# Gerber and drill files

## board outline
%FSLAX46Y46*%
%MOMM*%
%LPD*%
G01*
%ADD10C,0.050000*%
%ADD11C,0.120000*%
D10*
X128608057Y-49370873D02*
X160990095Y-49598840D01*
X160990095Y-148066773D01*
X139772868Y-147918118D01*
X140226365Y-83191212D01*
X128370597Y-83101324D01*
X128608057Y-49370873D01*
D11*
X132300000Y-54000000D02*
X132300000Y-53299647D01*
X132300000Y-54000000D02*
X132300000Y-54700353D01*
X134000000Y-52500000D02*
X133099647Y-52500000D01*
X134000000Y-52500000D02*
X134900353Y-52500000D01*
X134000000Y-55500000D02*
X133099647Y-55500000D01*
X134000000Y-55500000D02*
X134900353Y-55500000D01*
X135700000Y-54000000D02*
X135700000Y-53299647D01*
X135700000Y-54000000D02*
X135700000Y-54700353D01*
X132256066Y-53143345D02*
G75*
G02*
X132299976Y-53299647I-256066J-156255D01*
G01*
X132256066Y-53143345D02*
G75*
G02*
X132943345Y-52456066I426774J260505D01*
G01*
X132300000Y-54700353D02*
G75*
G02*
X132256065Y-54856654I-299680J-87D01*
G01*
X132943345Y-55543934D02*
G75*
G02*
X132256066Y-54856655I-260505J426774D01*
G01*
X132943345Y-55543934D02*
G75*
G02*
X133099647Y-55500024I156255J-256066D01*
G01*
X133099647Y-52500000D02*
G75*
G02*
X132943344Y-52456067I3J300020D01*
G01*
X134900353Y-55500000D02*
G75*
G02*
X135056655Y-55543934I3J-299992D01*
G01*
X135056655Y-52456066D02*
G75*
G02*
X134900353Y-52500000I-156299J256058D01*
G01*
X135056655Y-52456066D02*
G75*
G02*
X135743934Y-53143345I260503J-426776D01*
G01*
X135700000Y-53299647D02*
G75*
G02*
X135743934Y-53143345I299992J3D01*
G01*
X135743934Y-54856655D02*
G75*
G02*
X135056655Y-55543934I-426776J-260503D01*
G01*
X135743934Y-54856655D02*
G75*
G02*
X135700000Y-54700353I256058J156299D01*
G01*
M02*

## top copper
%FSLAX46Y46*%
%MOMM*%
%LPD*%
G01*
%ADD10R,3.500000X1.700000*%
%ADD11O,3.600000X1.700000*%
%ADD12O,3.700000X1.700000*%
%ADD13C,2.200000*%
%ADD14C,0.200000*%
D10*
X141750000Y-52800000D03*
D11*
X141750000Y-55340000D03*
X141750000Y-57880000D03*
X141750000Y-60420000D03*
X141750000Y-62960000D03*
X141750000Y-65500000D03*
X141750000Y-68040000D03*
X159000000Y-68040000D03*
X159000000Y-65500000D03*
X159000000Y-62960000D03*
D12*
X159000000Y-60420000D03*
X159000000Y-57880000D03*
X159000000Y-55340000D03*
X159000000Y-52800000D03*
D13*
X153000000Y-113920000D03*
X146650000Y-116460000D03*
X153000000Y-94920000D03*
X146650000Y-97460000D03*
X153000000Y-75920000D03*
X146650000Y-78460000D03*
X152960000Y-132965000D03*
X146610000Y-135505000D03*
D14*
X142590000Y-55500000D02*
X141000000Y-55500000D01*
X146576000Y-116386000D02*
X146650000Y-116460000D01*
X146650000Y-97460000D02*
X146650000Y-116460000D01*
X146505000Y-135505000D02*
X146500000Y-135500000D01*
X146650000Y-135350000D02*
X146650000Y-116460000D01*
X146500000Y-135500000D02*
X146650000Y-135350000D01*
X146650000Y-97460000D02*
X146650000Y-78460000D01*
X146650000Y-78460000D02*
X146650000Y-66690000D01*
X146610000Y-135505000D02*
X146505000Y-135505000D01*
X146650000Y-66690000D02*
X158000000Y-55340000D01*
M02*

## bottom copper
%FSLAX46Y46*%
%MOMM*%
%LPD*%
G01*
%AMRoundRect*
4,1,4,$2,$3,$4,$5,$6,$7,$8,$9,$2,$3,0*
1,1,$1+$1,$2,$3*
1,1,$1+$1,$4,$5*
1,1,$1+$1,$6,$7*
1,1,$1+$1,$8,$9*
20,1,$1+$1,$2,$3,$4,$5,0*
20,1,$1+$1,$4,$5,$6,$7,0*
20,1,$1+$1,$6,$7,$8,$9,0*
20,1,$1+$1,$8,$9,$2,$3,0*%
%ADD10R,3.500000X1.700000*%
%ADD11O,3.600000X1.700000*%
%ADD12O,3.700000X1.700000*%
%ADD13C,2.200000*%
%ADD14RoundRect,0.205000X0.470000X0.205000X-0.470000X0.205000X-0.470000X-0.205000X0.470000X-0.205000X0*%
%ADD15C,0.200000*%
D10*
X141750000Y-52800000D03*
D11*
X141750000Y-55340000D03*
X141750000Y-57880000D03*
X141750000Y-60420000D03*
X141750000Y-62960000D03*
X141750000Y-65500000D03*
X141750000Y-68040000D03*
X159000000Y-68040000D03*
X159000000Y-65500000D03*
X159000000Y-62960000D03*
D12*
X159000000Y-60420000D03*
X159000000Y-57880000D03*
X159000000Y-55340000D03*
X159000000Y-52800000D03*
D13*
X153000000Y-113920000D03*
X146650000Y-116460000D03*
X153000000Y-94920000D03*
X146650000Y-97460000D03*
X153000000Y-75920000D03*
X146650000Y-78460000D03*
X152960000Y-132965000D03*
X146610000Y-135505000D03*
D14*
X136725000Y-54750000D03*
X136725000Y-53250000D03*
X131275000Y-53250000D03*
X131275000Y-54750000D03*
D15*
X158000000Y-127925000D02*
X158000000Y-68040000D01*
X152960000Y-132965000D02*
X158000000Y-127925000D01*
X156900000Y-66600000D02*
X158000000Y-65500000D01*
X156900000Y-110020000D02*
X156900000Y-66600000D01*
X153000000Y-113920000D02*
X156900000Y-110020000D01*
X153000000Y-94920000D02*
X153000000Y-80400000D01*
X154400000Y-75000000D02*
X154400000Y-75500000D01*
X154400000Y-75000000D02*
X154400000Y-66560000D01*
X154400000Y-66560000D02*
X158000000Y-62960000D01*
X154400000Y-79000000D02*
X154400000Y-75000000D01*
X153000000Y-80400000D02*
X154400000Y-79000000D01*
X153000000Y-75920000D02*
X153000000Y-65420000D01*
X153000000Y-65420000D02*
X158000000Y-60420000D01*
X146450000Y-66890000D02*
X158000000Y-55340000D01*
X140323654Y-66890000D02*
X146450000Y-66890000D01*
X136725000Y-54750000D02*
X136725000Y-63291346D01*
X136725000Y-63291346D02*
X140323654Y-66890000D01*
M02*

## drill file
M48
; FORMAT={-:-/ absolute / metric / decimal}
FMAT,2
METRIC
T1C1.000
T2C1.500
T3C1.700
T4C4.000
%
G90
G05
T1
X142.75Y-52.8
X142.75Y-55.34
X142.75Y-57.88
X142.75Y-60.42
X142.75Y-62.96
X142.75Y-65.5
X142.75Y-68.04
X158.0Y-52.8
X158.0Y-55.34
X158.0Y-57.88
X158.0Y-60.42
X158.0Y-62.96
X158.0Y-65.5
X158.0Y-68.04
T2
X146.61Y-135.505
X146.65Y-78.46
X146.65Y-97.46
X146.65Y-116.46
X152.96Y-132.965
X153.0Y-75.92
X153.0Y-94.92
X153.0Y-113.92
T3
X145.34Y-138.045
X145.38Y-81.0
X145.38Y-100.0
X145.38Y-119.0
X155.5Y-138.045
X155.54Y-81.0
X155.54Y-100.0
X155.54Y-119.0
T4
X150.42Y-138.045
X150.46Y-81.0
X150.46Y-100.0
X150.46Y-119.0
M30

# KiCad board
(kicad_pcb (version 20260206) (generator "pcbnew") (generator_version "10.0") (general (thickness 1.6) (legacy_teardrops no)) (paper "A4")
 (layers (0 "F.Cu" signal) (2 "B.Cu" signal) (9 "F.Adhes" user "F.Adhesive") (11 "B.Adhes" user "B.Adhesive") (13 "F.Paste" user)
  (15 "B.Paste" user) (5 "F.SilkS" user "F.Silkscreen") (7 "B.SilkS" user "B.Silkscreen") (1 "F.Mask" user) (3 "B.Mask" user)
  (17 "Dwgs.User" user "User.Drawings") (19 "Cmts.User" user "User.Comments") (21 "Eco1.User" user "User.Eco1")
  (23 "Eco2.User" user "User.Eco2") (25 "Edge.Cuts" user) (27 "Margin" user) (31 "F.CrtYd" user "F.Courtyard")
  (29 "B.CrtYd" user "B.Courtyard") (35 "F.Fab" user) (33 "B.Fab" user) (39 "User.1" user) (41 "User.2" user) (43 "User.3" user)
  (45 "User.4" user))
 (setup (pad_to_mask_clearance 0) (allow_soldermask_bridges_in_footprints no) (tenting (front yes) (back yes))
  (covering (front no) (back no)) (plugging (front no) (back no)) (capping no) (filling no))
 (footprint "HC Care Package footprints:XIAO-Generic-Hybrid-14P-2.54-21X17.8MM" (layer "F.Cu") (at 150.375 60.42)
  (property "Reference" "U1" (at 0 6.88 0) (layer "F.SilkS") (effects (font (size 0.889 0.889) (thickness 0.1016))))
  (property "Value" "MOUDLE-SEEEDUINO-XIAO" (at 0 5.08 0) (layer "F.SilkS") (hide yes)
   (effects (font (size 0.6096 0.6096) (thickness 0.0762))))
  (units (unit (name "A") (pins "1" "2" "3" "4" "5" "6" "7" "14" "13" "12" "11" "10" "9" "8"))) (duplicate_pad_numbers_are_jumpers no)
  (pad "1" thru_hole rect (at -7.625 -7.62) (size 3.5 1.7) (drill 1 (offset -1 0)) (layers "*.Cu" "*.Mask") (remove_unused_layers no)
   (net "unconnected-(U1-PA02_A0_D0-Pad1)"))
  (pad "2" thru_hole oval (at -7.625 -5.08) (size 3.6 1.7) (drill 1 (offset -1 0)) (layers "*.Cu" "*.Mask") (remove_unused_layers no)
   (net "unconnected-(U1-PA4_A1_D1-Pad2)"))
  (pad "3" thru_hole oval (at -7.625 -2.54) (size 3.6 1.7) (drill 1 (offset -1 0)) (layers "*.Cu" "*.Mask") (remove_unused_layers no)
   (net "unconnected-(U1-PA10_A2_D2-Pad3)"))
  (pad "4" thru_hole oval (at -7.625 0) (size 3.6 1.7) (drill 1 (offset -1 0)) (layers "*.Cu" "*.Mask") (remove_unused_layers no)
   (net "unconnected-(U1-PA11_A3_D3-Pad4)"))
  (pad "5" thru_hole oval (at -7.625 2.54) (size 3.6 1.7) (drill 1 (offset -1 0)) (layers "*.Cu" "*.Mask") (remove_unused_layers no)
   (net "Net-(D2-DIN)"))
  (pad "6" thru_hole oval (at -7.625 5.08 180) (size 3.6 1.7) (drill 1 (offset 1 0)) (layers "*.Cu" "*.Mask") (remove_unused_layers no)
   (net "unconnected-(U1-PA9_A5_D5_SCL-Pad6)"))
  (pad "7" thru_hole oval (at -7.625 7.62) (size 3.6 1.7) (drill 1 (offset -1 0)) (layers "*.Cu" "*.Mask") (remove_unused_layers no)
   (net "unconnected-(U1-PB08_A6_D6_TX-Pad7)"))
  (pad "8" thru_hole oval (at 7.625 7.62) (size 3.6 1.7) (drill 1 (offset 1 0)) (layers "*.Cu" "*.Mask") (remove_unused_layers no)
   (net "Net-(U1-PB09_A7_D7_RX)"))
  (pad "9" thru_hole oval (at 7.625 5.08) (size 3.6 1.7) (drill 1 (offset 1 0)) (layers "*.Cu" "*.Mask") (remove_unused_layers no)
   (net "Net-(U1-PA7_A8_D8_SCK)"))
  (pad "10" thru_hole oval (at 7.625 2.54) (size 3.6 1.7) (drill 1 (offset 1 0)) (layers "*.Cu" "*.Mask") (remove_unused_layers no)
   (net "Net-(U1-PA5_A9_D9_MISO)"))
  (pad "11" thru_hole oval (at 7.625 0) (size 3.7 1.7) (drill 1 (offset 1 0)) (layers "*.Cu" "*.Mask") (remove_unused_layers no)
   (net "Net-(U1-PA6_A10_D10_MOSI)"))
  (pad "12" thru_hole oval (at 7.625 -2.54) (size 3.7 1.7) (drill 1 (offset 1 0)) (layers "*.Cu" "*.Mask") (remove_unused_layers no)
   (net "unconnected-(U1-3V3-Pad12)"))
  (pad "13" thru_hole oval (at 7.625 -5.08) (size 3.7 1.7) (drill 1 (offset 1 0)) (layers "*.Cu" "*.Mask") (remove_unused_layers no)
   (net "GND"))
  (pad "14" thru_hole oval (at 7.625 -7.62) (size 3.7 1.7) (drill 1 (offset 1 0)) (layers "*.Cu" "*.Mask") (remove_unused_layers no)
   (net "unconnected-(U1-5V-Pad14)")))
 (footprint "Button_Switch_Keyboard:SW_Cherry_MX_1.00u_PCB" (layer "F.Cu") (at 153 113.92)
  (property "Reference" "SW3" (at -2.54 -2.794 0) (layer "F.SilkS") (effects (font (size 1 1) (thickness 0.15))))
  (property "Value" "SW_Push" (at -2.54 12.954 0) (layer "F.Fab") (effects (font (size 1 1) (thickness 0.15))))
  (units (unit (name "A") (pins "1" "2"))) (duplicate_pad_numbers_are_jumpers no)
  (pad "" np_thru_hole circle (at -7.62 5.08) (size 1.7 1.7) (drill 1.7) (layers "*.Cu" "*.Mask"))
  (pad "" np_thru_hole circle (at -2.54 5.08) (size 4 4) (drill 4) (layers "*.Cu" "*.Mask"))
  (pad "" np_thru_hole circle (at 2.54 5.08) (size 1.7 1.7) (drill 1.7) (layers "*.Cu" "*.Mask"))
  (pad "1" thru_hole circle (at 0 0) (size 2.2 2.2) (drill 1.5) (layers "*.Cu" "*.Mask") (remove_unused_layers no)
   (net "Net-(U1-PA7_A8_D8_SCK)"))
  (pad "2" thru_hole circle (at -6.35 2.54) (size 2.2 2.2) (drill 1.5) (layers "*.Cu" "*.Mask") (remove_unused_layers no) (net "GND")))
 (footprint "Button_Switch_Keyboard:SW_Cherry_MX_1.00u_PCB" (layer "F.Cu") (at 153 94.92)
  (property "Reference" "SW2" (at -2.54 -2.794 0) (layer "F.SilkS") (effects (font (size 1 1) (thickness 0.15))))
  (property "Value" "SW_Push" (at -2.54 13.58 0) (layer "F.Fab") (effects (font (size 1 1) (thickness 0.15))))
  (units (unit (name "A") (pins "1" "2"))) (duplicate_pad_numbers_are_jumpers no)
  (pad "" np_thru_hole circle (at -7.62 5.08) (size 1.7 1.7) (drill 1.7) (layers "*.Cu" "*.Mask"))
  (pad "" np_thru_hole circle (at -2.54 5.08) (size 4 4) (drill 4) (layers "*.Cu" "*.Mask"))
  (pad "" np_thru_hole circle (at 2.54 5.08) (size 1.7 1.7) (drill 1.7) (layers "*.Cu" "*.Mask"))
  (pad "1" thru_hole circle (at 0 0) (size 2.2 2.2) (drill 1.5) (layers "*.Cu" "*.Mask") (remove_unused_layers no)
   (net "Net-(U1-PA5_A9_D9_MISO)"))
  (pad "2" thru_hole circle (at -6.35 2.54) (size 2.2 2.2) (drill 1.5) (layers "*.Cu" "*.Mask") (remove_unused_layers no) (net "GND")))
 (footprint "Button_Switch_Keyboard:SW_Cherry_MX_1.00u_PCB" (layer "F.Cu") (at 153 75.92)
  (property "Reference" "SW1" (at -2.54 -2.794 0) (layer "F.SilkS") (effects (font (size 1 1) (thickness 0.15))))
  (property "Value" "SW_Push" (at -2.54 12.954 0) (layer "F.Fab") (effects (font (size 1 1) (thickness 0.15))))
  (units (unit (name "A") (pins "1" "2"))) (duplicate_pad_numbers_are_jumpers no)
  (pad "" np_thru_hole circle (at -7.62 5.08) (size 1.7 1.7) (drill 1.7) (layers "*.Cu" "*.Mask"))
  (pad "" np_thru_hole circle (at -2.54 5.08) (size 4 4) (drill 4) (layers "*.Cu" "*.Mask"))
  (pad "" np_thru_hole circle (at 2.54 5.08) (size 1.7 1.7) (drill 1.7) (layers "*.Cu" "*.Mask"))
  (pad "1" thru_hole circle (at 0 0) (size 2.2 2.2) (drill 1.5) (layers "*.Cu" "*.Mask") (remove_unused_layers no)
   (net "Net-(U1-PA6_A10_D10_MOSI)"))
  (pad "2" thru_hole circle (at -6.35 2.54) (size 2.2 2.2) (drill 1.5) (layers "*.Cu" "*.Mask") (remove_unused_layers no) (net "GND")))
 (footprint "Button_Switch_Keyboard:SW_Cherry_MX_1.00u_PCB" (layer "F.Cu") (at 152.96 132.965)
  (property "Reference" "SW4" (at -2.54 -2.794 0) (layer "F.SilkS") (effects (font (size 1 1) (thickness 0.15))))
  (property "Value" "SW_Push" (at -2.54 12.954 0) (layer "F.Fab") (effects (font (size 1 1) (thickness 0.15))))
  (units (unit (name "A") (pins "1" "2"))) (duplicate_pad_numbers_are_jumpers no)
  (pad "" np_thru_hole circle (at -7.62 5.08) (size 1.7 1.7) (drill 1.7) (layers "*.Cu" "*.Mask"))
  (pad "" np_thru_hole circle (at -2.54 5.08) (size 4 4) (drill 4) (layers "*.Cu" "*.Mask"))
  (pad "" np_thru_hole circle (at 2.54 5.08) (size 1.7 1.7) (drill 1.7) (layers "*.Cu" "*.Mask"))
  (pad "1" thru_hole circle (at 0 0) (size 2.2 2.2) (drill 1.5) (layers "*.Cu" "*.Mask") (remove_unused_layers no)
   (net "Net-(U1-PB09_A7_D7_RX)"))
  (pad "2" thru_hole circle (at -6.35 2.54) (size 2.2 2.2) (drill 1.5) (layers "*.Cu" "*.Mask") (remove_unused_layers no) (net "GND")))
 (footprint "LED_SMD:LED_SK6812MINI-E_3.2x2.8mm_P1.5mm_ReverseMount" (layer "B.Cu") (at 134 54 180)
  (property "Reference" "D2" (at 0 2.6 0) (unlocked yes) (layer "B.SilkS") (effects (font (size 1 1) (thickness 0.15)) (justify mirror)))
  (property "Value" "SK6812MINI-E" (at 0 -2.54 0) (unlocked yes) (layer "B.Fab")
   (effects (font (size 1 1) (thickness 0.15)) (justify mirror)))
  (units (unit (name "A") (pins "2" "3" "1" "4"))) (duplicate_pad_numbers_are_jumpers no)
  (fp_line (start 1.7 0) (end 1.7 0.700353) (stroke (width 0.12) (type solid)) (layer "Edge.Cuts"))
  (fp_line (start 1.7 0) (end 1.7 -0.700353) (stroke (width 0.12) (type solid)) (layer "Edge.Cuts"))
  (fp_line (start 0 1.5) (end 0.900353 1.5) (stroke (width 0.12) (type solid)) (layer "Edge.Cuts"))
  (fp_line (start 0 1.5) (end -0.900353 1.5) (stroke (width 0.12) (type solid)) (layer "Edge.Cuts"))
  (fp_line (start 0 -1.5) (end 0.900353 -1.5) (stroke (width 0.12) (type solid)) (layer "Edge.Cuts"))
  (fp_line (start 0 -1.5) (end -0.900353 -1.5) (stroke (width 0.12) (type solid)) (layer "Edge.Cuts"))
  (fp_line (start -1.7 0) (end -1.7 0.700353) (stroke (width 0.12) (type solid)) (layer "Edge.Cuts"))
  (fp_line (start -1.7 0) (end -1.7 -0.700353) (stroke (width 0.12) (type solid)) (layer "Edge.Cuts"))
  (fp_arc (start 1.743934 0.856655) (mid 1.711191 0.781533) (end 1.7 0.700353) (stroke (width 0.12) (type solid)) (layer "Edge.Cuts"))
  (fp_arc (start 1.743934 0.856655) (mid 1.670713 1.470713) (end 1.056655 1.543934) (stroke (width 0.12) (type solid)) (layer "Edge.Cuts"))
  (fp_arc (start 1.7 -0.700353) (mid 1.711181 -0.781538) (end 1.743934 -0.856655) (stroke (width 0.12) (type solid)) (layer "Edge.Cuts"))
  (fp_arc (start 1.056655 -1.543934) (mid 1.670711 -1.470711) (end 1.743934 -0.856655) (stroke (width 0.12) (type solid))
   (layer "Edge.Cuts"))
  (fp_arc (start 1.056655 -1.543934) (mid 0.981533 -1.511191) (end 0.900353 -1.5) (stroke (width 0.12) (type solid)) (layer "Edge.Cuts"))
  (fp_arc (start 0.900353 1.5) (mid 0.981532 1.511193) (end 1.056655 1.543934) (stroke (width 0.12) (type solid)) (layer "Edge.Cuts"))
  (fp_arc (start -0.900353 -1.5) (mid -0.981533 -1.511192) (end -1.056655 -1.543934) (stroke (width 0.12) (type solid)) (layer "Edge.Cuts"))
  (fp_arc (start -1.056655 1.543934) (mid -0.981533 1.511192) (end -0.900353 1.5) (stroke (width 0.12) (type solid)) (layer "Edge.Cuts"))
  (fp_arc (start -1.056655 1.543934) (mid -1.670711 1.470711) (end -1.743934 0.856655) (stroke (width 0.12) (type solid))
   (layer "Edge.Cuts"))
  (fp_arc (start -1.7 0.700353) (mid -1.711192 0.781533) (end -1.743934 0.856655) (stroke (width 0.12) (type solid)) (layer "Edge.Cuts"))
  (fp_arc (start -1.743934 -0.856655) (mid -1.670711 -1.470711) (end -1.056655 -1.543934) (stroke (width 0.12) (type solid))
   (layer "Edge.Cuts"))
  (fp_arc (start -1.743934 -0.856655) (mid -1.711192 -0.781533) (end -1.7 -0.700353) (stroke (width 0.12) (type solid)) (layer "Edge.Cuts"))
  (pad "1" smd roundrect (at -2.725 -0.75 180) (size 1.35 0.82) (layers "B.Cu" "B.Mask" "B.Paste") (roundrect_rratio 0.25) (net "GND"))
  (pad "2" smd roundrect (at -2.725 0.75 180) (size 1.35 0.82) (layers "B.Cu" "B.Mask" "B.Paste") (roundrect_rratio 0.25)
   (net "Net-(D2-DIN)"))
  (pad "3" smd roundrect (at 2.725 0.75 180) (size 1.35 0.82) (layers "B.Cu" "B.Mask" "B.Paste") (roundrect_rratio 0.25) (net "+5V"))
  (pad "4" smd roundrect (at 2.725 -0.75 180) (size 1.35 0.82) (layers "B.Cu" "B.Mask" "B.Paste") (roundrect_rratio 0.25)
   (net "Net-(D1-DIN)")))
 (gr_poly
  (pts (xy 128.608057 49.370873) (xy 160.990095 49.59884) (xy 160.990095 148.066773) (xy 139.772868 147.918118) (xy 140.226365 83.191212)
   (xy 128.370597 83.101324))
  (stroke (width 0.05) (type solid)) (fill no) (layer "Edge.Cuts"))
 (segment (start 142.59 55.5) (end 141 55.5) (width 0.2) (layer "F.Cu") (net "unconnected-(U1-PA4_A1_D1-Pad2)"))
 (segment (start 158 127.925) (end 158 68.04) (width 0.2) (layer "B.Cu") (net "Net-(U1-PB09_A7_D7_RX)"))
 (segment (start 152.96 132.965) (end 158 127.925) (width 0.2) (layer "B.Cu") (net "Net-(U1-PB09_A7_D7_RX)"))
 (segment (start 156.9 66.6) (end 158 65.5) (width 0.2) (layer "B.Cu") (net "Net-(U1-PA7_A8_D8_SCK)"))
 (segment (start 156.9 110.02) (end 156.9 66.6) (width 0.2) (layer "B.Cu") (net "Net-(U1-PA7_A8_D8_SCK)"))
 (segment (start 153 113.92) (end 156.9 110.02) (width 0.2) (layer "B.Cu") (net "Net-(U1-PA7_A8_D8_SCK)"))
 (segment (start 153 94.92) (end 153 80.4) (width 0.2) (layer "B.Cu") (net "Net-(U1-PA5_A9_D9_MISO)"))
 (segment (start 154.4 75) (end 154.4 75.5) (width 0.2) (layer "B.Cu") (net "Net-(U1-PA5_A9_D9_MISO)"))
 (segment (start 154.4 75) (end 154.4 66.56) (width 0.2) (layer "B.Cu") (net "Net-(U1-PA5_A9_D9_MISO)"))
 (segment (start 154.4 66.56) (end 158 62.96) (width 0.2) (layer "B.Cu") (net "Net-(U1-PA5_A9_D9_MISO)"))
 (segment (start 154.4 79) (end 154.4 75) (width 0.2) (layer "B.Cu") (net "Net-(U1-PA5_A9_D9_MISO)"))
 (segment (start 153 80.4) (end 154.4 79) (width 0.2) (layer "B.Cu") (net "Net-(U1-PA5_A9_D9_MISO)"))
 (segment (start 153 75.92) (end 153 65.42) (width 0.2) (layer "B.Cu") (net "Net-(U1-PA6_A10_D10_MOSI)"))
 (segment (start 153 65.42) (end 158 60.42) (width 0.2) (layer "B.Cu") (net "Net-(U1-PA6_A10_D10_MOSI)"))
 (segment (start 146.576 116.386) (end 146.65 116.46) (width 0.2) (layer "F.Cu") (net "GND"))
 (segment (start 146.65 97.46) (end 146.65 116.46) (width 0.2) (layer "F.Cu") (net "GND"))
 (segment (start 146.505 135.505) (end 146.5 135.5) (width 0.2) (layer "F.Cu") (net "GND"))
 (segment (start 146.65 135.35) (end 146.65 116.46) (width 0.2) (layer "F.Cu") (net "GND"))
 (segment (start 146.5 135.5) (end 146.65 135.35) (width 0.2) (layer "F.Cu") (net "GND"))
 (segment (start 146.65 97.46) (end 146.65 78.46) (width 0.2) (layer "F.Cu") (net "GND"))
 (segment (start 146.65 78.46) (end 146.65 66.69) (width 0.2) (layer "F.Cu") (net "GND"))
 (segment (start 146.61 135.505) (end 146.505 135.505) (width 0.2) (layer "F.Cu") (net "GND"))
 (segment (start 146.65 66.69) (end 158 55.34) (width 0.2) (layer "F.Cu") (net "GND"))
 (segment (start 146.45 66.89) (end 158 55.34) (width 0.2) (layer "B.Cu") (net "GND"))
 (segment (start 140.323654 66.89) (end 146.45 66.89) (width 0.2) (layer "B.Cu") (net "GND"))
 (segment (start 136.725 54.75) (end 136.725 63.291346) (width 0.2) (layer "B.Cu") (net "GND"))
 (segment (start 136.725 63.291346) (end 140.323654 66.89) (width 0.2) (layer "B.Cu") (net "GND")))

